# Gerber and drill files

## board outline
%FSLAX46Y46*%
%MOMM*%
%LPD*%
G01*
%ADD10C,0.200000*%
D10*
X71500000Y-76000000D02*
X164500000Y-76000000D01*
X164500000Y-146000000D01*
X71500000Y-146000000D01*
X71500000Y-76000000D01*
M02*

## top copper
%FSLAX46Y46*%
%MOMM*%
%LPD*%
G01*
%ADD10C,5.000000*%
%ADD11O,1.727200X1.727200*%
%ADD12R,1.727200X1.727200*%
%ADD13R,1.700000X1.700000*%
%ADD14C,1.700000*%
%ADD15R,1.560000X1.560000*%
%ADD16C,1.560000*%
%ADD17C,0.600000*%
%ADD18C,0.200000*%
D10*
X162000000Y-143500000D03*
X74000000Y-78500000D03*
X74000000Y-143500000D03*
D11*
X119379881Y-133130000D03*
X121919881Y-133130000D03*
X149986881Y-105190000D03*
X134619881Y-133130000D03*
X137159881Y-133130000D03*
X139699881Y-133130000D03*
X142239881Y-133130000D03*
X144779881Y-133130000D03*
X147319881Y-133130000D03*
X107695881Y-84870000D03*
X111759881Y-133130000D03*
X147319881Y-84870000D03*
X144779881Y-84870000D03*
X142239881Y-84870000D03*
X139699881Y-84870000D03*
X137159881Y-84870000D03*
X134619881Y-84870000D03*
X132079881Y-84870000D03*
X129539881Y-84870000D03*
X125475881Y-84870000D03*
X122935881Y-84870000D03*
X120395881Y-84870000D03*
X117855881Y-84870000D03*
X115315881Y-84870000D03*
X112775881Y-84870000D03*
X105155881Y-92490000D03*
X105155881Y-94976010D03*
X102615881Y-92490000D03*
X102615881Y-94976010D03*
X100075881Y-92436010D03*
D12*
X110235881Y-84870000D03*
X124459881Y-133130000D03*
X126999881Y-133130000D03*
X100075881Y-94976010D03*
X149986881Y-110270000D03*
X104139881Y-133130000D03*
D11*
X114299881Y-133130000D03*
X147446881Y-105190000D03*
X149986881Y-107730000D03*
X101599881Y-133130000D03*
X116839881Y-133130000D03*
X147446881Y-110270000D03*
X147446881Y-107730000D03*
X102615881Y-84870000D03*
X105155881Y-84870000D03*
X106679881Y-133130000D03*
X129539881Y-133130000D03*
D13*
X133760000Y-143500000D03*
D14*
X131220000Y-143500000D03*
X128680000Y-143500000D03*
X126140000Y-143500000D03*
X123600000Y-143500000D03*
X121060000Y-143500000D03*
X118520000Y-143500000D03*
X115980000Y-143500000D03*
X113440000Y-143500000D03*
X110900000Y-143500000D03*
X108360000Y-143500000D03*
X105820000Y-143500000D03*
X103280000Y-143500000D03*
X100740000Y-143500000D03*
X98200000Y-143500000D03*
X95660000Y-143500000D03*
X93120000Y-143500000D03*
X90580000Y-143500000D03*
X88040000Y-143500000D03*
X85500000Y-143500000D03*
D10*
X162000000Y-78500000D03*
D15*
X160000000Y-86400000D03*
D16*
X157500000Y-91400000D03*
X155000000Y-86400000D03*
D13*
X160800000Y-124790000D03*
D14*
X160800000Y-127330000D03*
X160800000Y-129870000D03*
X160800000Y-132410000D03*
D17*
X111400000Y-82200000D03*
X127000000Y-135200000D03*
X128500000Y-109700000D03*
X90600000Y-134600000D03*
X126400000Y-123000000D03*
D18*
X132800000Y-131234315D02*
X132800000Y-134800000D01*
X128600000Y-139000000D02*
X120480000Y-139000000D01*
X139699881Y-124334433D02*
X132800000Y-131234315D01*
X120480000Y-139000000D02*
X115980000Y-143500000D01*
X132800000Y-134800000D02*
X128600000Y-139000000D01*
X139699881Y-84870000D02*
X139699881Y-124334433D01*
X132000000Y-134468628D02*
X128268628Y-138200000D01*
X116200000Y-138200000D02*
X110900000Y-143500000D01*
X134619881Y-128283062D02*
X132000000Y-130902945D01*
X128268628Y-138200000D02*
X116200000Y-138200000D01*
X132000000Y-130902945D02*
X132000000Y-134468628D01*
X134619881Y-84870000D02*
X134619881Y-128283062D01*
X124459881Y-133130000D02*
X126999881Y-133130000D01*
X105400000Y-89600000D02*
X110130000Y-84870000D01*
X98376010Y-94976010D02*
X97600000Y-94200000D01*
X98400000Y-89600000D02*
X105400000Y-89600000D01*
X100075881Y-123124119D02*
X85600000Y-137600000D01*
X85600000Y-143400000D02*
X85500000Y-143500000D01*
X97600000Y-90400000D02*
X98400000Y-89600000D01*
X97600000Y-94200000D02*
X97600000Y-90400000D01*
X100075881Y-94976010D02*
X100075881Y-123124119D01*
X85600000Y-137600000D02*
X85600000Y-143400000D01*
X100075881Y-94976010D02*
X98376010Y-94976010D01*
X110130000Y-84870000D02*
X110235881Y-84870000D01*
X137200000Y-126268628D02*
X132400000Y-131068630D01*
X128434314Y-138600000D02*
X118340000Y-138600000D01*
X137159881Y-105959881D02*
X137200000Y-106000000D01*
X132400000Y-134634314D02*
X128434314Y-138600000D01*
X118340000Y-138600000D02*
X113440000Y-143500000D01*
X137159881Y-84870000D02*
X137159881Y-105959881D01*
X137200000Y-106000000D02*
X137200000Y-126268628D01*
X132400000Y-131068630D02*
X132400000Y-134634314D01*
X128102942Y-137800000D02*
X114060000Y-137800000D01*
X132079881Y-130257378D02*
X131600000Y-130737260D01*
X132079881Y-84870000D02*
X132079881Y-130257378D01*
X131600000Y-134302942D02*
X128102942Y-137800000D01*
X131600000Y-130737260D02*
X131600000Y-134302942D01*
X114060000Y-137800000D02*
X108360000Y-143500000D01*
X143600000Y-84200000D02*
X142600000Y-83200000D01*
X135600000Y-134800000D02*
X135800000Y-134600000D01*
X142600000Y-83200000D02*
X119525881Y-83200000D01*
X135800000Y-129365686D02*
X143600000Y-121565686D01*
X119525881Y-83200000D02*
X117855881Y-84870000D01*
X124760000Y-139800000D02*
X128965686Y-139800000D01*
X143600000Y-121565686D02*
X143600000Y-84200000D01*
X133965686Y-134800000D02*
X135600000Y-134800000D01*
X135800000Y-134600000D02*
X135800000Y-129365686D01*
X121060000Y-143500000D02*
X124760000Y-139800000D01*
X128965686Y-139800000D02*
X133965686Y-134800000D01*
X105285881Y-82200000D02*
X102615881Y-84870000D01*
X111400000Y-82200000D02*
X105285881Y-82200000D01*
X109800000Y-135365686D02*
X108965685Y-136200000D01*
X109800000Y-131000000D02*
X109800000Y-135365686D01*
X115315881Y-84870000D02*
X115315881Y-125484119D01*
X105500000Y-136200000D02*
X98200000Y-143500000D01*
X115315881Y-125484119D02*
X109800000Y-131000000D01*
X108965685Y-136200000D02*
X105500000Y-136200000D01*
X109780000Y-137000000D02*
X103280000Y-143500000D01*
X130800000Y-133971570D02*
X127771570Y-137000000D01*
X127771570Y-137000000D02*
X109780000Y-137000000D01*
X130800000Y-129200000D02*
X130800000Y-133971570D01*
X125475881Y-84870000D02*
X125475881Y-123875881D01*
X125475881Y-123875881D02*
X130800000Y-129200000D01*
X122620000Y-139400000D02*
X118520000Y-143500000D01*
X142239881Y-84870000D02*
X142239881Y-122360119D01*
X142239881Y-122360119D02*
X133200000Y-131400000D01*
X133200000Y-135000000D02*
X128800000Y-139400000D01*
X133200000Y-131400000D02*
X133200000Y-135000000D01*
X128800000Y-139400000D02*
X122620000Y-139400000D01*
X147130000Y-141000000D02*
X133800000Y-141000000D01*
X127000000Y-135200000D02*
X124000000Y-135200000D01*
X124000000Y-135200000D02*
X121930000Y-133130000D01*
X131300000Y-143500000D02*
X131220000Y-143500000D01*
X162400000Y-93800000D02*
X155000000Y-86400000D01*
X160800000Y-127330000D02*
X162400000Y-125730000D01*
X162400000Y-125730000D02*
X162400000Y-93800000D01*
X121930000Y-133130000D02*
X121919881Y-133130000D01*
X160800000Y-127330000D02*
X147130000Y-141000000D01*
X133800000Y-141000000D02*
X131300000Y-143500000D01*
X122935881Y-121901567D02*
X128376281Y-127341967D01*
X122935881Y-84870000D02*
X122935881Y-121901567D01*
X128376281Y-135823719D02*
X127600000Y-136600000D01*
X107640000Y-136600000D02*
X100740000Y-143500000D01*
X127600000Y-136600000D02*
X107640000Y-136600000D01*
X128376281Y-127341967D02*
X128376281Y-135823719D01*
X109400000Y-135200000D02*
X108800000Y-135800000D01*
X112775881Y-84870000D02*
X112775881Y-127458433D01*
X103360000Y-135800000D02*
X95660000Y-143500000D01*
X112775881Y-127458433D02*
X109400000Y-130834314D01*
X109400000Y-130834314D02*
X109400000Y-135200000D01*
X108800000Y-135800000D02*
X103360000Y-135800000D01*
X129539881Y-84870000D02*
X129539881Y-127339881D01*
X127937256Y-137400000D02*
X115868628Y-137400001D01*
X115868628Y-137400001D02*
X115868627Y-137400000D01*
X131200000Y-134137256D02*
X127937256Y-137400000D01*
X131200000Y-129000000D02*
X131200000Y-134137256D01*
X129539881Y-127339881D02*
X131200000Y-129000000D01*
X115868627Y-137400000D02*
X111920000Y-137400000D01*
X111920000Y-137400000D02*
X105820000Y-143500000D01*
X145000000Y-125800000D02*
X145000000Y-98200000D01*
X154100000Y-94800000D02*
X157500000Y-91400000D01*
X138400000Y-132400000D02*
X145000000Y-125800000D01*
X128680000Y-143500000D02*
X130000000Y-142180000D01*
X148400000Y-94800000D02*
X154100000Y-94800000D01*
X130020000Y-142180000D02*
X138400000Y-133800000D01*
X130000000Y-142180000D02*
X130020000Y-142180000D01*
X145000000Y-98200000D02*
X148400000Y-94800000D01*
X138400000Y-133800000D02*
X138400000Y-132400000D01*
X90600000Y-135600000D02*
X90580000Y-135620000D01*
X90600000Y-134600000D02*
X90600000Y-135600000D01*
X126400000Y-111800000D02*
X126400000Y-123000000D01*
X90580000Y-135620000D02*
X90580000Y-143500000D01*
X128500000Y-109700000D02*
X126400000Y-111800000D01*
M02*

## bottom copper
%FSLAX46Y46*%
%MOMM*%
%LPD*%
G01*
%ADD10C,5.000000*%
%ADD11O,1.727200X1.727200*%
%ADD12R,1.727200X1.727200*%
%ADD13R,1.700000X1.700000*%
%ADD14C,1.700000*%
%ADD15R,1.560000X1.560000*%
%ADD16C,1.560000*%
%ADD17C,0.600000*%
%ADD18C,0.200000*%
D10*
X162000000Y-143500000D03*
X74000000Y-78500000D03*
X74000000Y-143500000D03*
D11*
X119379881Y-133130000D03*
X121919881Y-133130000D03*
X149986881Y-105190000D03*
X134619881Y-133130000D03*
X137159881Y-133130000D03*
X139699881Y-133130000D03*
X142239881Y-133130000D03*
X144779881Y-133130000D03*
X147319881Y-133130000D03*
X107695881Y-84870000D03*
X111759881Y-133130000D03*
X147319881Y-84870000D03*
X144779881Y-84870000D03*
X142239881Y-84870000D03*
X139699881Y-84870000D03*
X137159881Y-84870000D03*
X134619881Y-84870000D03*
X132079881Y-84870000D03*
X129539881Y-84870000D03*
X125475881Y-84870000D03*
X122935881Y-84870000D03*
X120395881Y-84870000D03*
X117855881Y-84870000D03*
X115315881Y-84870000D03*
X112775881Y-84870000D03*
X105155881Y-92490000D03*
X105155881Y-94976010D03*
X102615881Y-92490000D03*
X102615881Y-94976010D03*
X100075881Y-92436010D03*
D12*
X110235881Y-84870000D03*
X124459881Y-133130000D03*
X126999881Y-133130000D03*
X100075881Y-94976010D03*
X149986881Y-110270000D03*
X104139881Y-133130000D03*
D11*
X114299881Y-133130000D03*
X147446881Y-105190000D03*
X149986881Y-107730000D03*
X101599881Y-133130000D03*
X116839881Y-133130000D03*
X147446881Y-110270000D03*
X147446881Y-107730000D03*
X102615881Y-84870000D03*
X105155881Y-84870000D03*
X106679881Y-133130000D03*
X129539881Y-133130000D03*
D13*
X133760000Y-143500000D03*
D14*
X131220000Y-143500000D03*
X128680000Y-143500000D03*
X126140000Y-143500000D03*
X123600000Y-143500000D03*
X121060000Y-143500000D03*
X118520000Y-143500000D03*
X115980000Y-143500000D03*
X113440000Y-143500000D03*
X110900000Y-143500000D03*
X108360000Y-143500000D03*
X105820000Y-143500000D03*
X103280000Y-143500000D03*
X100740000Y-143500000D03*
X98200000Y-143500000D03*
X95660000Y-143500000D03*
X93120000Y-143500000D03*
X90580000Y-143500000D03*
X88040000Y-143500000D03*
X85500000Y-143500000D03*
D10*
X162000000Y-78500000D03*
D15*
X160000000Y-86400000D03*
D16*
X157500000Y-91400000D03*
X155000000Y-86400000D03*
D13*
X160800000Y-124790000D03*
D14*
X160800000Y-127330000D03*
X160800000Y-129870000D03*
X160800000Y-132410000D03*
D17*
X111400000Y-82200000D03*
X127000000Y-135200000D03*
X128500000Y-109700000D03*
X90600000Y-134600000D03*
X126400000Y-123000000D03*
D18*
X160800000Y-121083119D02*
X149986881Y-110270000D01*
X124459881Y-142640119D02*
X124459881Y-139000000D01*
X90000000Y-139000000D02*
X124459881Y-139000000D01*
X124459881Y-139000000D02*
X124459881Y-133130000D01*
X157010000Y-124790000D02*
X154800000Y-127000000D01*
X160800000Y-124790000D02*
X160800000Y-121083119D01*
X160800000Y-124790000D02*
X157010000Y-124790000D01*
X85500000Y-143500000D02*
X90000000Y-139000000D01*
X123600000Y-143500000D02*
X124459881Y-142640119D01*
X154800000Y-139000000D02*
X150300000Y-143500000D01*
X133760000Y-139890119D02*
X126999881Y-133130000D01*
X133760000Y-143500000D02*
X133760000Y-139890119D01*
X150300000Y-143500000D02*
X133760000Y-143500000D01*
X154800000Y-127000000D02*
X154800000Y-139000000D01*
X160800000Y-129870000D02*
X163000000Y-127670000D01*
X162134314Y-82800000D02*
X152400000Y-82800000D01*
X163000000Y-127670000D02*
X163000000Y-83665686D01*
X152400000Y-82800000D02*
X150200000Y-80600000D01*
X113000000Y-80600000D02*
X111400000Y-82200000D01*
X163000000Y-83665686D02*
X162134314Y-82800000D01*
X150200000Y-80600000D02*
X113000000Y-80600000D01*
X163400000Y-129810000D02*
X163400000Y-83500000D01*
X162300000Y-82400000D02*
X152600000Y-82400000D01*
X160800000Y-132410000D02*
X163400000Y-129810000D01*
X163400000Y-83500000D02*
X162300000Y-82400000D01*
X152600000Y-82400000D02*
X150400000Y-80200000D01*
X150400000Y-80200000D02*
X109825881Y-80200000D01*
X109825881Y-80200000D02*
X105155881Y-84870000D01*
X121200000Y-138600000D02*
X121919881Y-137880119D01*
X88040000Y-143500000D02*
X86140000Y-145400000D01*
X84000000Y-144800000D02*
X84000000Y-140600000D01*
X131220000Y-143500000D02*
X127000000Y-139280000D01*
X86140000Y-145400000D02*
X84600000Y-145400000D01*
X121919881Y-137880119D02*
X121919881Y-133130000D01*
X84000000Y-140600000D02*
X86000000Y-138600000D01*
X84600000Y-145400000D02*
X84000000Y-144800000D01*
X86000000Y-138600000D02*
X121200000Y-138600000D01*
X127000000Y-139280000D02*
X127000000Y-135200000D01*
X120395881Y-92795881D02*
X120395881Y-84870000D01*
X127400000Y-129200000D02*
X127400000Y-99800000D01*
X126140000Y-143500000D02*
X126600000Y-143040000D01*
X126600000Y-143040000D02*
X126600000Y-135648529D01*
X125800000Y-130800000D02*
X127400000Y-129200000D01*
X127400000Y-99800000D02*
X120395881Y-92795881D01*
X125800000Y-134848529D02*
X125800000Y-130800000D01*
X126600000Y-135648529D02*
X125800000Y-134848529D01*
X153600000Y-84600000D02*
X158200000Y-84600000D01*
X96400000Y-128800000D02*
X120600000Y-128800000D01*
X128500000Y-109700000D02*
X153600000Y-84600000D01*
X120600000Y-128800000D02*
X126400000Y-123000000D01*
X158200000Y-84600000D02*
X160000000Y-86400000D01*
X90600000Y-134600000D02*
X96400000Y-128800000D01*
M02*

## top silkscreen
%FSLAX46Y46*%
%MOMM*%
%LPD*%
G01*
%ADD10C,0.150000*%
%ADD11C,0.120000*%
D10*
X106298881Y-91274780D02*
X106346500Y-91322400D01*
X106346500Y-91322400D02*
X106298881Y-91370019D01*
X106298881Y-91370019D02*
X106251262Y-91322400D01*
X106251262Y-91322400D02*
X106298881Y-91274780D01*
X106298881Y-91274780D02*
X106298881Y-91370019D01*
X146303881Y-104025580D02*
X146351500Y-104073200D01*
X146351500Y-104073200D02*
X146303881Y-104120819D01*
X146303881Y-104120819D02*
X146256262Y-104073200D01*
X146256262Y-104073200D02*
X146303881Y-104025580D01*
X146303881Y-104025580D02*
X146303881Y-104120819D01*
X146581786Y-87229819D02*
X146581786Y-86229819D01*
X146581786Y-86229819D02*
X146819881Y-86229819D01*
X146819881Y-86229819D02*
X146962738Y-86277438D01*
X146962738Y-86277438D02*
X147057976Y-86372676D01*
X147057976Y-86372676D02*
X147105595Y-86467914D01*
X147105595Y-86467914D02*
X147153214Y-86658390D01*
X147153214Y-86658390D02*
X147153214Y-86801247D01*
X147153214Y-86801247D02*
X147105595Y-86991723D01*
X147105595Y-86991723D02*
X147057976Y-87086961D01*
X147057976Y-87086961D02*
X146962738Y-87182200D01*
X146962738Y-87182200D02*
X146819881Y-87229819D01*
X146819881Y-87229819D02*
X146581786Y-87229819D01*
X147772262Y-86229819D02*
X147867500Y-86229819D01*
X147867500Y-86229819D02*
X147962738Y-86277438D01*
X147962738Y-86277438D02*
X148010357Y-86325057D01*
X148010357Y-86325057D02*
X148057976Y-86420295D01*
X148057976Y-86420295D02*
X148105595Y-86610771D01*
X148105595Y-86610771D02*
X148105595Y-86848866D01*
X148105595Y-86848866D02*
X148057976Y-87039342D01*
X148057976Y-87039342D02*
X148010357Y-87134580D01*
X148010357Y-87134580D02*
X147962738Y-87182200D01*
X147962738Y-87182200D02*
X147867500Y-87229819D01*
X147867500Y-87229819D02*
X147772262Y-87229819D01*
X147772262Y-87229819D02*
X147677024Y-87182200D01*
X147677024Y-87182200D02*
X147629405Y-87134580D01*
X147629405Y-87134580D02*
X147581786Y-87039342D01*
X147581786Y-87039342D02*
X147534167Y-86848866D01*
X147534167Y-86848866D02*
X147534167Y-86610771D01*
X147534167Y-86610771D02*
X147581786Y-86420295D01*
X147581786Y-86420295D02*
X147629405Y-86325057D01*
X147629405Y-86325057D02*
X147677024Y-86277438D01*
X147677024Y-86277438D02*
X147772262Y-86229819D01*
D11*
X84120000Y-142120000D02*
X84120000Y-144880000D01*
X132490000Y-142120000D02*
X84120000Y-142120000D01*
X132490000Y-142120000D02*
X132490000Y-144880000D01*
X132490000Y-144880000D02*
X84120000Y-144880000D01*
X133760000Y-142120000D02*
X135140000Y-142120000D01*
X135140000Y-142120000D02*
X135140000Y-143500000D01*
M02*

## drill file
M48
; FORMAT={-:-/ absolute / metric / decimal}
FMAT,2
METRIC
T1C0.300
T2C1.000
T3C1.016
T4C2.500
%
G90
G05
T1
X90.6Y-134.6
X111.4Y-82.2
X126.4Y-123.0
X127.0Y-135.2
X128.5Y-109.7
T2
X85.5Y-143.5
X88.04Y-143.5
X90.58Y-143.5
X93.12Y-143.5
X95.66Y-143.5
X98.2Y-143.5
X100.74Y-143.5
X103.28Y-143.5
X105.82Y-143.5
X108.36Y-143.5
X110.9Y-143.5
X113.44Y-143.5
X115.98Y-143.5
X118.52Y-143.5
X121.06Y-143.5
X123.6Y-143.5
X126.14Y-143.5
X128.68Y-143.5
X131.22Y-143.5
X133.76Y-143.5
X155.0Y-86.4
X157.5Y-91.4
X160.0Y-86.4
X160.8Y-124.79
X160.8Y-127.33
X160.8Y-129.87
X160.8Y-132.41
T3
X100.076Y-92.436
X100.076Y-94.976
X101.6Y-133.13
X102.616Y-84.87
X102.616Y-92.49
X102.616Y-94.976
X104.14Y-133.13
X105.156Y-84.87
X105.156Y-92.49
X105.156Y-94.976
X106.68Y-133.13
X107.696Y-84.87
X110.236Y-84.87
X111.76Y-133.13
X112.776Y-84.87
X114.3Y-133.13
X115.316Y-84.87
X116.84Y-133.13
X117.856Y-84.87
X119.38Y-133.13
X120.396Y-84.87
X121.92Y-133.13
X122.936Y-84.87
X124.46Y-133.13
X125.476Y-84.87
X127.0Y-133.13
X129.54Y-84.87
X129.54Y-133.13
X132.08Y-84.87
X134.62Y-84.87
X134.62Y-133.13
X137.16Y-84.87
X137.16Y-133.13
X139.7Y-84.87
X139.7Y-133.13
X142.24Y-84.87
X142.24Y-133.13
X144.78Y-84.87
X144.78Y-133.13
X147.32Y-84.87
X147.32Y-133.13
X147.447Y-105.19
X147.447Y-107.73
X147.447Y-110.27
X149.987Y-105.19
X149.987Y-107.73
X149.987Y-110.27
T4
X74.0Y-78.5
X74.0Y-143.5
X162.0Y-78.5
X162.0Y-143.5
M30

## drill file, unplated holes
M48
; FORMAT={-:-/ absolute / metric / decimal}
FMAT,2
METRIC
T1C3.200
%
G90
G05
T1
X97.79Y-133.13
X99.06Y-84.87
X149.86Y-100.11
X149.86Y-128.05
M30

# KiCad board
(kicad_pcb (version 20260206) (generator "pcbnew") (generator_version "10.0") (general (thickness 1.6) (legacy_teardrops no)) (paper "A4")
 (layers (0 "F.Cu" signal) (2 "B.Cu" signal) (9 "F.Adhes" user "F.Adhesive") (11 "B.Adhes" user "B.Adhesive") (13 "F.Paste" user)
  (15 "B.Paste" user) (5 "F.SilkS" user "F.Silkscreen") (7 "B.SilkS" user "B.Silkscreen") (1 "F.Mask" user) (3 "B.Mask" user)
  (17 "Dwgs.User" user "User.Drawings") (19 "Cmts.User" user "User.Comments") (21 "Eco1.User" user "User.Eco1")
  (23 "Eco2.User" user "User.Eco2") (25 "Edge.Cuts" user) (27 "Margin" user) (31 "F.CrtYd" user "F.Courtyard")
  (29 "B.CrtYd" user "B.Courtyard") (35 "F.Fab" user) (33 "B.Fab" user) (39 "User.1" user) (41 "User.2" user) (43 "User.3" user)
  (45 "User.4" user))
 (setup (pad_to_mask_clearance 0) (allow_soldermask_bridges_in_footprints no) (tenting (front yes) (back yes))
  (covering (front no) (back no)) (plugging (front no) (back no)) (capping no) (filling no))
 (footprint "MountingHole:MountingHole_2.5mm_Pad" (layer "F.Cu") (at 162 143.5)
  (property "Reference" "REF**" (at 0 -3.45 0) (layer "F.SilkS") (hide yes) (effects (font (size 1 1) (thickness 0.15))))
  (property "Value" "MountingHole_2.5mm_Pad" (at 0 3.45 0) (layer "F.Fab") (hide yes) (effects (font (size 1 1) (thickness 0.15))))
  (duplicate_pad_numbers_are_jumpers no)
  (pad "1" thru_hole circle (at 0 0) (size 5 5) (drill 2.5) (layers "*.Cu" "*.Mask") (remove_unused_layers no) (zone_connect 2)))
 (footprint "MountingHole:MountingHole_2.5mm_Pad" (layer "F.Cu") (at 74 78.5)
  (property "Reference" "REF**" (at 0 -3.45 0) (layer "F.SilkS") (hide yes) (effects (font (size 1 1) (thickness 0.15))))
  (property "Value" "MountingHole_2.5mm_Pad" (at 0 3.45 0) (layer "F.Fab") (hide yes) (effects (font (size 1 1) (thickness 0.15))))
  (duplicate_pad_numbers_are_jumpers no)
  (pad "1" thru_hole circle (at 0 0) (size 5 5) (drill 2.5) (layers "*.Cu" "*.Mask") (remove_unused_layers no) (zone_connect 2)))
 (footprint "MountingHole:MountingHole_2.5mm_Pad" (layer "F.Cu") (at 74 143.5)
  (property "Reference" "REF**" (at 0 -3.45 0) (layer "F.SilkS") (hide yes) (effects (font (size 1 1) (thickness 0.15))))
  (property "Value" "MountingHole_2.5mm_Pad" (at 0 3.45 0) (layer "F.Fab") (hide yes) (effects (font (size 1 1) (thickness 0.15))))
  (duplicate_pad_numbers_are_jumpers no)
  (pad "1" thru_hole circle (at 0 0) (size 5 5) (drill 2.5) (layers "*.Cu" "*.Mask") (remove_unused_layers no) (zone_connect 2)))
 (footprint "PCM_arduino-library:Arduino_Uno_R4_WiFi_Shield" (layer "F.Cu") (at 83.819881 135.67)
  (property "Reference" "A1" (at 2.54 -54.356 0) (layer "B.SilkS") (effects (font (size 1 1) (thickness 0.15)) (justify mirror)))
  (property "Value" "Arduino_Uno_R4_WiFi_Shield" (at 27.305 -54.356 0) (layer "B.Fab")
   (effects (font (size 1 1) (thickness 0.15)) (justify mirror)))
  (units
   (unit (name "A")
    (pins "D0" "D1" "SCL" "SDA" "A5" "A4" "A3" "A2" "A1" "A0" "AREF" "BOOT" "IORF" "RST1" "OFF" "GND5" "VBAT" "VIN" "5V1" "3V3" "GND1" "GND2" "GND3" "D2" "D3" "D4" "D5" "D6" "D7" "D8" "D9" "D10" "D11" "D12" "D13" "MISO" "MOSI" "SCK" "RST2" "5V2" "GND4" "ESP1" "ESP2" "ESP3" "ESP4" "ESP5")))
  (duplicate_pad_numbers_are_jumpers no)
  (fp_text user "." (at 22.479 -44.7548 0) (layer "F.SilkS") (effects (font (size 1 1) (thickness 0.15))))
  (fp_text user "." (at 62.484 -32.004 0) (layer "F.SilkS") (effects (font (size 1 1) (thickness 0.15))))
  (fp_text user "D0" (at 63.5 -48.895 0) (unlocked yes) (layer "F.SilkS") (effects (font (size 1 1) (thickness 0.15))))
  (pad "" np_thru_hole circle (at 13.97 -2.54) (size 3.2 3.2) (drill 3.2) (layers "*.Cu" "*.Mask"))
  (pad "" np_thru_hole circle (at 15.24 -50.8) (size 3.2 3.2) (drill 3.2) (layers "*.Cu" "*.Mask"))
  (pad "" np_thru_hole circle (at 66.04 -35.56) (size 3.2 3.2) (drill 3.2) (layers "*.Cu" "*.Mask"))
  (pad "" np_thru_hole circle (at 66.04 -7.62) (size 3.2 3.2) (drill 3.2) (layers "*.Cu" "*.Mask"))
  (pad "3V3" thru_hole oval (at 35.56 -2.54) (size 1.7272 1.7272) (drill 1.016) (layers "*.Cu" "*.Mask") (remove_unused_layers no)
   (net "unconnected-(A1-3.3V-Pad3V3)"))
  (pad "5V1" thru_hole oval (at 38.1 -2.54) (size 1.7272 1.7272) (drill 1.016) (layers "*.Cu" "*.Mask") (remove_unused_layers no)
   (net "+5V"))
  (pad "5V2" thru_hole oval (at 66.167 -30.48) (size 1.7272 1.7272) (drill 1.016) (layers "*.Cu" "*.Mask") (remove_unused_layers no)
   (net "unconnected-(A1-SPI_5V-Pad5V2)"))
  (pad "A0" thru_hole oval (at 50.8 -2.54) (size 1.7272 1.7272) (drill 1.016) (layers "*.Cu" "*.Mask") (remove_unused_layers no)
   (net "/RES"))
  (pad "A1" thru_hole oval (at 53.34 -2.54) (size 1.7272 1.7272) (drill 1.016) (layers "*.Cu" "*.Mask") (remove_unused_layers no)
   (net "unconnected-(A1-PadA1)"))
  (pad "A2" thru_hole oval (at 55.88 -2.54) (size 1.7272 1.7272) (drill 1.016) (layers "*.Cu" "*.Mask") (remove_unused_layers no)
   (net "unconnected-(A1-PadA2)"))
  (pad "A3" thru_hole oval (at 58.42 -2.54) (size 1.7272 1.7272) (drill 1.016) (layers "*.Cu" "*.Mask") (remove_unused_layers no)
   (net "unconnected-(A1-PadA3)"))
  (pad "A4" thru_hole oval (at 60.96 -2.54) (size 1.7272 1.7272) (drill 1.016) (layers "*.Cu" "*.Mask") (remove_unused_layers no)
   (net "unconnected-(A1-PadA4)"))
  (pad "A5" thru_hole oval (at 63.5 -2.54) (size 1.7272 1.7272) (drill 1.016) (layers "*.Cu" "*.Mask") (remove_unused_layers no)
   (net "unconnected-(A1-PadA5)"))
  (pad "AREF" thru_hole oval (at 23.876 -50.8) (size 1.7272 1.7272) (drill 1.016) (layers "*.Cu" "*.Mask") (remove_unused_layers no)
   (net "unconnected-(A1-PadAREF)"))
  (pad "BOOT" thru_hole oval (at 27.94 -2.54) (size 1.7272 1.7272) (drill 1.016) (layers "*.Cu" "*.Mask") (remove_unused_layers no)
   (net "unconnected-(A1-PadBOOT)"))
  (pad "D0" thru_hole oval (at 63.5 -50.8) (size 1.7272 1.7272) (drill 1.016) (layers "*.Cu" "*.Mask") (remove_unused_layers no)
   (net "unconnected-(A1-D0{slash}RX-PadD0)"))
  (pad "D1" thru_hole oval (at 60.96 -50.8) (size 1.7272 1.7272) (drill 1.016) (layers "*.Cu" "*.Mask") (remove_unused_layers no)
   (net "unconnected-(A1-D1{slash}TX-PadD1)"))
  (pad "D2" thru_hole oval (at 58.42 -50.8) (size 1.7272 1.7272) (drill 1.016) (layers "*.Cu" "*.Mask") (remove_unused_layers no)
   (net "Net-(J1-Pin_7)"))
  (pad "D3" thru_hole oval (at 55.88 -50.8) (size 1.7272 1.7272) (drill 1.016) (layers "*.Cu" "*.Mask") (remove_unused_layers no)
   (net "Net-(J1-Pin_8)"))
  (pad "D4" thru_hole oval (at 53.34 -50.8) (size 1.7272 1.7272) (drill 1.016) (layers "*.Cu" "*.Mask") (remove_unused_layers no)
   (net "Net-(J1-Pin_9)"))
  (pad "D5" thru_hole oval (at 50.8 -50.8) (size 1.7272 1.7272) (drill 1.016) (layers "*.Cu" "*.Mask") (remove_unused_layers no)
   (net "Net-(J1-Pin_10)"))
  (pad "D6" thru_hole oval (at 48.26 -50.8) (size 1.7272 1.7272) (drill 1.016) (layers "*.Cu" "*.Mask") (remove_unused_layers no)
   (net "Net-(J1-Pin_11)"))
  (pad "D7" thru_hole oval (at 45.72 -50.8) (size 1.7272 1.7272) (drill 1.016) (layers "*.Cu" "*.Mask") (remove_unused_layers no)
   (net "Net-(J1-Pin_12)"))
  (pad "D8" thru_hole oval (at 41.656 -50.8) (size 1.7272 1.7272) (drill 1.016) (layers "*.Cu" "*.Mask") (remove_unused_layers no)
   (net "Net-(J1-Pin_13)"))
  (pad "D9" thru_hole oval (at 39.116 -50.8) (size 1.7272 1.7272) (drill 1.016) (layers "*.Cu" "*.Mask") (remove_unused_layers no)
   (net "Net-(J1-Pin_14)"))
  (pad "D10" thru_hole oval (at 36.576 -50.8) (size 1.7272 1.7272) (drill 1.016) (layers "*.Cu" "*.Mask") (remove_unused_layers no)
   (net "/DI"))
  (pad "D11" thru_hole oval (at 34.036 -50.8) (size 1.7272 1.7272) (drill 1.016) (layers "*.Cu" "*.Mask") (remove_unused_layers no)
   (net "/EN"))
  (pad "D12" thru_hole oval (at 31.496 -50.8) (size 1.7272 1.7272) (drill 1.016) (layers "*.Cu" "*.Mask") (remove_unused_layers no)
   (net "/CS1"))
  (pad "D13" thru_hole oval (at 28.956 -50.8) (size 1.7272 1.7272) (drill 1.016) (layers "*.Cu" "*.Mask") (remove_unused_layers no)
   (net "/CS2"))
  (pad "ESP1" thru_hole oval (at 21.336 -43.18) (size 1.7272 1.7272) (drill 1.016) (layers "*.Cu" "*.Mask") (remove_unused_layers no)
   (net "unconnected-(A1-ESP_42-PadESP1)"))
  (pad "ESP2" thru_hole oval (at 21.336 -40.69399) (size 1.7272 1.7272) (drill 1.016) (layers "*.Cu" "*.Mask") (remove_unused_layers no)
   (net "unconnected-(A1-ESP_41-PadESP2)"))
  (pad "ESP3" thru_hole oval (at 18.796 -43.18) (size 1.7272 1.7272) (drill 1.016) (layers "*.Cu" "*.Mask") (remove_unused_layers no)
   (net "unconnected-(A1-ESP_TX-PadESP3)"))
  (pad "ESP4" thru_hole oval (at 18.796 -40.69399) (size 1.7272 1.7272) (drill 1.016) (layers "*.Cu" "*.Mask") (remove_unused_layers no)
   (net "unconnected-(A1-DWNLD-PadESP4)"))
  (pad "ESP5" thru_hole oval (at 16.256 -43.23399) (size 1.7272 1.7272) (drill 1.016) (layers "*.Cu" "*.Mask") (remove_unused_layers no)
   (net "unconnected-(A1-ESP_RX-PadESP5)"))
  (pad "GND1" thru_hole rect (at 26.416 -50.8) (size 1.7272 1.7272) (drill 1.016) (layers "*.Cu" "*.Mask") (remove_unused_layers no)
   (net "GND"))
  (pad "GND2" thru_hole rect (at 40.64 -2.54) (size 1.7272 1.7272) (drill 1.016) (layers "*.Cu" "*.Mask") (remove_unused_layers no)
   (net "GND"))
  (pad "GND3" thru_hole rect (at 43.18 -2.54) (size 1.7272 1.7272) (drill 1.016) (layers "*.Cu" "*.Mask") (remove_unused_layers no)
   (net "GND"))
  (pad "GND4" thru_hole rect (at 16.256 -40.69399) (size 1.7272 1.7272) (drill 1.016) (layers "*.Cu" "*.Mask") (remove_unused_layers no)
   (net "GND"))
  (pad "GND4" thru_hole rect (at 66.167 -25.4) (size 1.7272 1.7272) (drill 1.016) (layers "*.Cu" "*.Mask") (remove_unused_layers no)
   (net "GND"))
  (pad "GND5" thru_hole rect (at 20.32 -2.54) (size 1.7272 1.7272) (drill 1.016) (layers "*.Cu" "*.Mask") (remove_unused_layers no)
   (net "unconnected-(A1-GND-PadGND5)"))
  (pad "IORF" thru_hole oval (at 30.48 -2.54) (size 1.7272 1.7272) (drill 1.016) (layers "*.Cu" "*.Mask") (remove_unused_layers no)
   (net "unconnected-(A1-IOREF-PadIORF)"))
  (pad "MISO" thru_hole oval (at 63.627 -30.48) (size 1.7272 1.7272) (drill 1.016) (layers "*.Cu" "*.Mask") (remove_unused_layers no)
   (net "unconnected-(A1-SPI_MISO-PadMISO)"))
  (pad "MOSI" thru_hole oval (at 66.167 -27.94) (size 1.7272 1.7272) (drill 1.016) (layers "*.Cu" "*.Mask") (remove_unused_layers no)
   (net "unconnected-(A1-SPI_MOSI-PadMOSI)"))
  (pad "OFF" thru_hole oval (at 17.78 -2.54) (size 1.7272 1.7272) (drill 1.016) (layers "*.Cu" "*.Mask") (remove_unused_layers no)
   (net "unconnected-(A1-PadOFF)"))
  (pad "RST1" thru_hole oval (at 33.02 -2.54) (size 1.7272 1.7272) (drill 1.016) (layers "*.Cu" "*.Mask") (remove_unused_layers no)
   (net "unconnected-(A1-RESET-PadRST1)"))
  (pad "RST2" thru_hole oval (at 63.627 -25.4) (size 1.7272 1.7272) (drill 1.016) (layers "*.Cu" "*.Mask") (remove_unused_layers no)
   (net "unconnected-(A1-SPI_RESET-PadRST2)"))
  (pad "SCK" thru_hole oval (at 63.627 -27.94) (size 1.7272 1.7272) (drill 1.016) (layers "*.Cu" "*.Mask") (remove_unused_layers no)
   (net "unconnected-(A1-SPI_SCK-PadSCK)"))
  (pad "SCL" thru_hole oval (at 18.796 -50.8) (size 1.7272 1.7272) (drill 1.016) (layers "*.Cu" "*.Mask") (remove_unused_layers no)
   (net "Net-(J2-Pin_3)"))
  (pad "SDA" thru_hole oval (at 21.336 -50.8) (size 1.7272 1.7272) (drill 1.016) (layers "*.Cu" "*.Mask") (remove_unused_layers no)
   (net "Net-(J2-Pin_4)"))
  (pad "VBAT" thru_hole oval (at 22.86 -2.54) (size 1.7272 1.7272) (drill 1.016) (layers "*.Cu" "*.Mask") (remove_unused_layers no)
   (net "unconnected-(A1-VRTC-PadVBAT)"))
  (pad "VIN" thru_hole oval (at 45.72 -2.54) (size 1.7272 1.7272) (drill 1.016) (layers "*.Cu" "*.Mask") (remove_unused_layers no)
   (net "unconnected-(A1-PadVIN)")))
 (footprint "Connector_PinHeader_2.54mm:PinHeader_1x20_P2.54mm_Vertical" (layer "F.Cu") (at 133.76 143.5 -90)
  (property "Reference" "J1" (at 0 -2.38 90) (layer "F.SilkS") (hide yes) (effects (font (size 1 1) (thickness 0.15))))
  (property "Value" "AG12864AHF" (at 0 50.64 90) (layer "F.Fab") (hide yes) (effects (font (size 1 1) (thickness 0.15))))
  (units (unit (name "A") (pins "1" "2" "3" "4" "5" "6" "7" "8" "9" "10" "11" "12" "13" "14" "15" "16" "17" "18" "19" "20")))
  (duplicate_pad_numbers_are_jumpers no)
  (fp_line (start -1.38 49.64) (end 1.38 49.64) (stroke (width 0.12) (type solid)) (layer "F.SilkS"))
  (fp_line (start -1.38 1.27) (end -1.38 49.64) (stroke (width 0.12) (type solid)) (layer "F.SilkS"))
  (fp_line (start -1.38 1.27) (end 1.38 1.27) (stroke (width 0.12) (type solid)) (layer "F.SilkS"))
  (fp_line (start 1.38 1.27) (end 1.38 49.64) (stroke (width 0.12) (type solid)) (layer "F.SilkS"))
  (fp_line (start -1.38 0) (end -1.38 -1.38) (stroke (width 0.12) (type solid)) (layer "F.SilkS"))
  (fp_line (start -1.38 -1.38) (end 0 -1.38) (stroke (width 0.12) (type solid)) (layer "F.SilkS"))
  (pad "1" thru_hole rect (at 0 0 270) (size 1.7 1.7) (drill 1) (layers "*.Cu" "*.Mask") (remove_unused_layers no) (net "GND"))
  (pad "2" thru_hole circle (at 0 2.54 270) (size 1.7 1.7) (drill 1) (layers "*.Cu" "*.Mask") (remove_unused_layers no) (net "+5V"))
  (pad "3" thru_hole circle (at 0 5.08 270) (size 1.7 1.7) (drill 1) (layers "*.Cu" "*.Mask") (remove_unused_layers no) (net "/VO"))
  (pad "4" thru_hole circle (at 0 7.62 270) (size 1.7 1.7) (drill 1) (layers "*.Cu" "*.Mask") (remove_unused_layers no) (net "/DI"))
  (pad "5" thru_hole circle (at 0 10.16 270) (size 1.7 1.7) (drill 1) (layers "*.Cu" "*.Mask") (remove_unused_layers no) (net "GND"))
  (pad "6" thru_hole circle (at 0 12.7 270) (size 1.7 1.7) (drill 1) (layers "*.Cu" "*.Mask") (remove_unused_layers no) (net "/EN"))
  (pad "7" thru_hole circle (at 0 15.24 270) (size 1.7 1.7) (drill 1) (layers "*.Cu" "*.Mask") (remove_unused_layers no)
   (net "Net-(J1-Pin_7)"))
  (pad "8" thru_hole circle (at 0 17.78 270) (size 1.7 1.7) (drill 1) (layers "*.Cu" "*.Mask") (remove_unused_layers no)
   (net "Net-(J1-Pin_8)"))
  (pad "9" thru_hole circle (at 0 20.32 270) (size 1.7 1.7) (drill 1) (layers "*.Cu" "*.Mask") (remove_unused_layers no)
   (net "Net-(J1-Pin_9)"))
  (pad "10" thru_hole circle (at 0 22.86 270) (size 1.7 1.7) (drill 1) (layers "*.Cu" "*.Mask") (remove_unused_layers no)
   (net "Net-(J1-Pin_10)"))
  (pad "11" thru_hole circle (at 0 25.4 270) (size 1.7 1.7) (drill 1) (layers "*.Cu" "*.Mask") (remove_unused_layers no)
   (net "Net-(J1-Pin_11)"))
  (pad "12" thru_hole circle (at 0 27.94 270) (size 1.7 1.7) (drill 1) (layers "*.Cu" "*.Mask") (remove_unused_layers no)
   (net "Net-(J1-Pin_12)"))
  (pad "13" thru_hole circle (at 0 30.48 270) (size 1.7 1.7) (drill 1) (layers "*.Cu" "*.Mask") (remove_unused_layers no)
   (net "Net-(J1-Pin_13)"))
  (pad "14" thru_hole circle (at 0 33.02 270) (size 1.7 1.7) (drill 1) (layers "*.Cu" "*.Mask") (remove_unused_layers no)
   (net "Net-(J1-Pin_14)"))
  (pad "15" thru_hole circle (at 0 35.56 270) (size 1.7 1.7) (drill 1) (layers "*.Cu" "*.Mask") (remove_unused_layers no) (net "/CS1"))
  (pad "16" thru_hole circle (at 0 38.1 270) (size 1.7 1.7) (drill 1) (layers "*.Cu" "*.Mask") (remove_unused_layers no) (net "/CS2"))
  (pad "17" thru_hole circle (at 0 40.64 270) (size 1.7 1.7) (drill 1) (layers "*.Cu" "*.Mask") (remove_unused_layers no) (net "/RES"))
  (pad "18" thru_hole circle (at 0 43.18 270) (size 1.7 1.7) (drill 1) (layers "*.Cu" "*.Mask") (remove_unused_layers no) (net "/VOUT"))
  (pad "19" thru_hole circle (at 0 45.72 270) (size 1.7 1.7) (drill 1) (layers "*.Cu" "*.Mask") (remove_unused_layers no) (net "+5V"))
  (pad "20" thru_hole circle (at 0 48.26 270) (size 1.7 1.7) (drill 1) (layers "*.Cu" "*.Mask") (remove_unused_layers no) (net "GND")))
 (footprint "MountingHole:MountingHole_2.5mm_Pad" (layer "F.Cu") (at 162 78.5)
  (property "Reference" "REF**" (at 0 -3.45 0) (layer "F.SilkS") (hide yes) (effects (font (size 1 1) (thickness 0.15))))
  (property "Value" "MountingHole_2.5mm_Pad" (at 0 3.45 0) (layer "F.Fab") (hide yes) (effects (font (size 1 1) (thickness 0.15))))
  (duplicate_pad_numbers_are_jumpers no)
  (pad "1" thru_hole circle (at 0 0) (size 5 5) (drill 2.5) (layers "*.Cu" "*.Mask") (remove_unused_layers no) (zone_connect 2)))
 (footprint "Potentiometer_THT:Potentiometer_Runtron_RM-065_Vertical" (layer "B.Cu") (at 160 86.4 180)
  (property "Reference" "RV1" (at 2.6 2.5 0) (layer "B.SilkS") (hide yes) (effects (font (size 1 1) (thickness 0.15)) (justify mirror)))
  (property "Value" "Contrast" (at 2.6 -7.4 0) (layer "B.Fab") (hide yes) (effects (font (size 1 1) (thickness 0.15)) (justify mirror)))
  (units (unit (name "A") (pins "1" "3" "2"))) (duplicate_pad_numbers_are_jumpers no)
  (pad "1" thru_hole rect (at 0 0 180) (size 1.56 1.56) (drill 1) (layers "*.Cu" "*.Mask") (remove_unused_layers no) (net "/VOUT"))
  (pad "2" thru_hole circle (at 2.5 -5 180) (size 1.56 1.56) (drill 1) (layers "*.Cu" "*.Mask") (remove_unused_layers no) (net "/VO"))
  (pad "3" thru_hole circle (at 5 0 180) (size 1.56 1.56) (drill 1) (layers "*.Cu" "*.Mask") (remove_unused_layers no) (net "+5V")))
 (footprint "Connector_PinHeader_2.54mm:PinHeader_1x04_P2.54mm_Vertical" (layer "B.Cu") (at 160.8 124.79 180)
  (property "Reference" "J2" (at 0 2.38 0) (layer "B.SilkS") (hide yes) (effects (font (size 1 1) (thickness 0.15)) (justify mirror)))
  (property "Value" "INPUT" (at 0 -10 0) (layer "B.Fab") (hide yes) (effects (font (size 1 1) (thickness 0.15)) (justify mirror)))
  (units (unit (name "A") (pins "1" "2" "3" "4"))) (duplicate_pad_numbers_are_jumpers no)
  (pad "1" thru_hole rect (at 0 0 180) (size 1.7 1.7) (drill 1) (layers "*.Cu" "*.Mask") (remove_unused_layers no) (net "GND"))
  (pad "2" thru_hole circle (at 0 -2.54 180) (size 1.7 1.7) (drill 1) (layers "*.Cu" "*.Mask") (remove_unused_layers no) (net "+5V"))
  (pad "3" thru_hole circle (at 0 -5.08 180) (size 1.7 1.7) (drill 1) (layers "*.Cu" "*.Mask") (remove_unused_layers no)
   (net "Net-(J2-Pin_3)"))
  (pad "4" thru_hole circle (at 0 -7.62 180) (size 1.7 1.7) (drill 1) (layers "*.Cu" "*.Mask") (remove_unused_layers no)
   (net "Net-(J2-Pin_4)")))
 (gr_rect (start 71.5 76) (end 164.5 146) (stroke (width 0.2) (type solid)) (fill no) (layer "Edge.Cuts"))
 (segment (start 147.13 141) (end 133.8 141) (width 0.2) (layer "F.Cu") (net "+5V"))
 (segment (start 127 135.2) (end 124 135.2) (width 0.2) (layer "F.Cu") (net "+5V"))
 (segment (start 124 135.2) (end 121.93 133.13) (width 0.2) (layer "F.Cu") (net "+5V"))
 (segment (start 131.3 143.5) (end 131.22 143.5) (width 0.2) (layer "F.Cu") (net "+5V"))
 (segment (start 162.4 93.8) (end 155 86.4) (width 0.2) (layer "F.Cu") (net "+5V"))
 (segment (start 160.8 127.33) (end 162.4 125.73) (width 0.2) (layer "F.Cu") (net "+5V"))
 (segment (start 162.4 125.73) (end 162.4 93.8) (width 0.2) (layer "F.Cu") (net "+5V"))
 (segment (start 121.93 133.13) (end 121.919881 133.13) (width 0.2) (layer "F.Cu") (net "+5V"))
 (segment (start 160.8 127.33) (end 147.13 141) (width 0.2) (layer "F.Cu") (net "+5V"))
 (segment (start 133.8 141) (end 131.3 143.5) (width 0.2) (layer "F.Cu") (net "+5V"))
 (via (at 127 135.2) (size 0.6) (drill 0.3) (layers "F.Cu" "B.Cu") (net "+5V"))
 (segment (start 121.2 138.6) (end 121.919881 137.880119) (width 0.2) (layer "B.Cu") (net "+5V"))
 (segment (start 88.04 143.5) (end 86.14 145.4) (width 0.2) (layer "B.Cu") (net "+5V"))
 (segment (start 84 144.8) (end 84 140.6) (width 0.2) (layer "B.Cu") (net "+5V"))
 (segment (start 131.22 143.5) (end 127 139.28) (width 0.2) (layer "B.Cu") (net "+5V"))
 (segment (start 86.14 145.4) (end 84.6 145.4) (width 0.2) (layer "B.Cu") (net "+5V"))
 (segment (start 121.919881 137.880119) (end 121.919881 133.13) (width 0.2) (layer "B.Cu") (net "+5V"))
 (segment (start 84 140.6) (end 86 138.6) (width 0.2) (layer "B.Cu") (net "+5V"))
 (segment (start 84.6 145.4) (end 84 144.8) (width 0.2) (layer "B.Cu") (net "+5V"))
 (segment (start 86 138.6) (end 121.2 138.6) (width 0.2) (layer "B.Cu") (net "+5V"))
 (segment (start 127 139.28) (end 127 135.2) (width 0.2) (layer "B.Cu") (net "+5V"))
 (segment (start 122.62 139.4) (end 118.52 143.5) (width 0.2) (layer "F.Cu") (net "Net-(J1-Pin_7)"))
 (segment (start 142.239881 84.87) (end 142.239881 122.360119) (width 0.2) (layer "F.Cu") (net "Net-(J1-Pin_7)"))
 (segment (start 142.239881 122.360119) (end 133.2 131.4) (width 0.2) (layer "F.Cu") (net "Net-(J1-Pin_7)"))
 (segment (start 133.2 135) (end 128.8 139.4) (width 0.2) (layer "F.Cu") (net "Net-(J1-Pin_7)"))
 (segment (start 133.2 131.4) (end 133.2 135) (width 0.2) (layer "F.Cu") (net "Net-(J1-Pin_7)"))
 (segment (start 128.8 139.4) (end 122.62 139.4) (width 0.2) (layer "F.Cu") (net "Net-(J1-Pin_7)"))
 (segment (start 132.8 131.234315) (end 132.8 134.8) (width 0.2) (layer "F.Cu") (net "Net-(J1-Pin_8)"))
 (segment (start 128.6 139) (end 120.48 139) (width 0.2) (layer "F.Cu") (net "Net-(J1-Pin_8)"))
 (segment (start 139.699881 124.334433) (end 132.8 131.234315) (width 0.2) (layer "F.Cu") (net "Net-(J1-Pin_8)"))
 (segment (start 120.48 139) (end 115.98 143.5) (width 0.2) (layer "F.Cu") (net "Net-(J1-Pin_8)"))
 (segment (start 132.8 134.8) (end 128.6 139) (width 0.2) (layer "F.Cu") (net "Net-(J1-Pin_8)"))
 (segment (start 139.699881 84.87) (end 139.699881 124.334433) (width 0.2) (layer "F.Cu") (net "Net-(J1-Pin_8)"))
 (segment (start 137.2 126.268628) (end 132.4 131.06863) (width 0.2) (layer "F.Cu") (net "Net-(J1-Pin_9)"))
 (segment (start 128.434314 138.6) (end 118.34 138.6) (width 0.2) (layer "F.Cu") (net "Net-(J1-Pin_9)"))
 (segment (start 137.159881 105.959881) (end 137.2 106) (width 0.2) (layer "F.Cu") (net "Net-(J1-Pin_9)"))
 (segment (start 132.4 134.634314) (end 128.434314 138.6) (width 0.2) (layer "F.Cu") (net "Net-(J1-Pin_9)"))
 (segment (start 118.34 138.6) (end 113.44 143.5) (width 0.2) (layer "F.Cu") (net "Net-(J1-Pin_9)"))
 (segment (start 137.159881 84.87) (end 137.159881 105.959881) (width 0.2) (layer "F.Cu") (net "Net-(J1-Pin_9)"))
 (segment (start 137.2 106) (end 137.2 126.268628) (width 0.2) (layer "F.Cu") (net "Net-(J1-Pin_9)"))
 (segment (start 132.4 131.06863) (end 132.4 134.634314) (width 0.2) (layer "F.Cu") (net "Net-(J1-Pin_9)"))
 (segment (start 132 134.468628) (end 128.268628 138.2) (width 0.2) (layer "F.Cu") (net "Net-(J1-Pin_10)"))
 (segment (start 116.2 138.2) (end 110.9 143.5) (width 0.2) (layer "F.Cu") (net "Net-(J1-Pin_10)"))
 (segment (start 134.619881 128.283062) (end 132 130.902945) (width 0.2) (layer "F.Cu") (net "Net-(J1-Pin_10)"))
 (segment (start 128.268628 138.2) (end 116.2 138.2) (width 0.2) (layer "F.Cu") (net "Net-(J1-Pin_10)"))
 (segment (start 132 130.902945) (end 132 134.468628) (width 0.2) (layer "F.Cu") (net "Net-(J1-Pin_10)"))
 (segment (start 134.619881 84.87) (end 134.619881 128.283062) (width 0.2) (layer "F.Cu") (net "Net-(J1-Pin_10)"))
 (segment (start 128.102942 137.8) (end 114.06 137.8) (width 0.2) (layer "F.Cu") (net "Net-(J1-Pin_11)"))
 (segment (start 132.079881 130.257378) (end 131.6 130.73726) (width 0.2) (layer "F.Cu") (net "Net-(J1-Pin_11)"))
 (segment (start 132.079881 84.87) (end 132.079881 130.257378) (width 0.2) (layer "F.Cu") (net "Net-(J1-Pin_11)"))
 (segment (start 131.6 134.302942) (end 128.102942 137.8) (width 0.2) (layer "F.Cu") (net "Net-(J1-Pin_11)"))
 (segment (start 131.6 130.73726) (end 131.6 134.302942) (width 0.2) (layer "F.Cu") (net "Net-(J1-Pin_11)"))
 (segment (start 114.06 137.8) (end 108.36 143.5) (width 0.2) (layer "F.Cu") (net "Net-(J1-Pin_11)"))
 (segment (start 129.539881 84.87) (end 129.539881 127.339881) (width 0.2) (layer "F.Cu") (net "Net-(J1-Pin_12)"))
 (segment (start 127.937256 137.4) (end 115.868628 137.400001) (width 0.2) (layer "F.Cu") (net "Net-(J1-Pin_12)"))
 (segment (start 115.868628 137.400001) (end 115.868627 137.4) (width 0.2) (layer "F.Cu") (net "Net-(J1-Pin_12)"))
 (segment (start 131.2 134.137256) (end 127.937256 137.4) (width 0.2) (layer "F.Cu") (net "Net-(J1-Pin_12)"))
 (segment (start 131.2 129) (end 131.2 134.137256) (width 0.2) (layer "F.Cu") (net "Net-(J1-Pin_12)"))
 (segment (start 129.539881 127.339881) (end 131.2 129) (width 0.2) (layer "F.Cu") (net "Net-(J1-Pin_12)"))
 (segment (start 115.868627 137.4) (end 111.92 137.4) (width 0.2) (layer "F.Cu") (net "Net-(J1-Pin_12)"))
 (segment (start 111.92 137.4) (end 105.82 143.5) (width 0.2) (layer "F.Cu") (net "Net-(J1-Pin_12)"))
 (segment (start 109.78 137) (end 103.28 143.5) (width 0.2) (layer "F.Cu") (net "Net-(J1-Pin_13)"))
 (segment (start 130.8 133.97157) (end 127.77157 137) (width 0.2) (layer "F.Cu") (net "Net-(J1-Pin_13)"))
 (segment (start 127.77157 137) (end 109.78 137) (width 0.2) (layer "F.Cu") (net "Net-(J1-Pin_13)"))
 (segment (start 130.8 129.2) (end 130.8 133.97157) (width 0.2) (layer "F.Cu") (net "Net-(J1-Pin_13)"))
 (segment (start 125.475881 84.87) (end 125.475881 123.875881) (width 0.2) (layer "F.Cu") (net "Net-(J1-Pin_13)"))
 (segment (start 125.475881 123.875881) (end 130.8 129.2) (width 0.2) (layer "F.Cu") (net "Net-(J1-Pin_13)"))
 (segment (start 122.935881 121.901567) (end 128.376281 127.341967) (width 0.2) (layer "F.Cu") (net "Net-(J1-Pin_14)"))
 (segment (start 122.935881 84.87) (end 122.935881 121.901567) (width 0.2) (layer "F.Cu") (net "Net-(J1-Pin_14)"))
 (segment (start 128.376281 135.823719) (end 127.6 136.6) (width 0.2) (layer "F.Cu") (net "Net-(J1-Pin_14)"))
 (segment (start 107.64 136.6) (end 100.74 143.5) (width 0.2) (layer "F.Cu") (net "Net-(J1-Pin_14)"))
 (segment (start 127.6 136.6) (end 107.64 136.6) (width 0.2) (layer "F.Cu") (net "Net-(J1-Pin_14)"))
 (segment (start 128.376281 127.341967) (end 128.376281 135.823719) (width 0.2) (layer "F.Cu") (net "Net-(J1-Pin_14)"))
 (segment (start 120.395881 92.795881) (end 120.395881 84.87) (width 0.2) (layer "B.Cu") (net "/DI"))
 (segment (start 127.4 129.2) (end 127.4 99.8) (width 0.2) (layer "B.Cu") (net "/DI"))
 (segment (start 126.14 143.5) (end 126.6 143.04) (width 0.2) (layer "B.Cu") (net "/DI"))
 (segment (start 126.6 143.04) (end 126.6 135.648529) (width 0.2) (layer "B.Cu") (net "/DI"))
 (segment (start 125.8 130.8) (end 127.4 129.2) (width 0.2) (layer "B.Cu") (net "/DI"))
 (segment (start 127.4 99.8) (end 120.395881 92.795881) (width 0.2) (layer "B.Cu") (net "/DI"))
 (segment (start 125.8 134.848529) (end 125.8 130.8) (width 0.2) (layer "B.Cu") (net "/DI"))
 (segment (start 126.6 135.648529) (end 125.8 134.848529) (width 0.2) (layer "B.Cu") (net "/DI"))
 (segment (start 143.6 84.2) (end 142.6 83.2) (width 0.2) (layer "F.Cu") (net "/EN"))
 (segment (start 135.6 134.8) (end 135.8 134.6) (width 0.2) (layer "F.Cu") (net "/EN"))
 (segment (start 142.6 83.2) (end 119.525881 83.2) (width 0.2) (layer "F.Cu") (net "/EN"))
 (segment (start 135.8 129.365686) (end 143.6 121.565686) (width 0.2) (layer "F.Cu") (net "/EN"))
 (segment (start 119.525881 83.2) (end 117.855881 84.87) (width 0.2) (layer "F.Cu") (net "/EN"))
 (segment (start 124.76 139.8) (end 128.965686 139.8) (width 0.2) (layer "F.Cu") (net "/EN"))
 (segment (start 143.6 121.565686) (end 143.6 84.2) (width 0.2) (layer "F.Cu") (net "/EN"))
 (segment (start 133.965686 134.8) (end 135.6 134.8) (width 0.2) (layer "F.Cu") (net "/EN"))
 (segment (start 135.8 134.6) (end 135.8 129.365686) (width 0.2) (layer "F.Cu") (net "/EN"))
 (segment (start 121.06 143.5) (end 124.76 139.8) (width 0.2) (layer "F.Cu") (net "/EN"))
 (segment (start 128.965686 139.8) (end 133.965686 134.8) (width 0.2) (layer "F.Cu") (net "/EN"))
 (segment (start 109.8 135.365686) (end 108.965685 136.2) (width 0.2) (layer "F.Cu") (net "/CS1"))
 (segment (start 109.8 131) (end 109.8 135.365686) (width 0.2) (layer "F.Cu") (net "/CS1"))
 (segment (start 115.315881 84.87) (end 115.315881 125.484119) (width 0.2) (layer "F.Cu") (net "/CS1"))
 (segment (start 105.5 136.2) (end 98.2 143.5) (width 0.2) (layer "F.Cu") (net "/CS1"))
 (segment (start 115.315881 125.484119) (end 109.8 131) (width 0.2) (layer "F.Cu") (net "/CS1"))
 (segment (start 108.965685 136.2) (end 105.5 136.2) (width 0.2) (layer "F.Cu") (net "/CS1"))
 (segment (start 109.4 135.2) (end 108.8 135.8) (width 0.2) (layer "F.Cu") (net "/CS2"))
 (segment (start 112.775881 84.87) (end 112.775881 127.458433) (width 0.2) (layer "F.Cu") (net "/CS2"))
 (segment (start 103.36 135.8) (end 95.66 143.5) (width 0.2) (layer "F.Cu") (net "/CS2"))
 (segment (start 112.775881 127.458433) (end 109.4 130.834314) (width 0.2) (layer "F.Cu") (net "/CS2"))
 (segment (start 109.4 130.834314) (end 109.4 135.2) (width 0.2) (layer "F.Cu") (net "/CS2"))
 (segment (start 108.8 135.8) (end 103.36 135.8) (width 0.2) (layer "F.Cu") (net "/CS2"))
 (segment (start 124.459881 133.13) (end 126.999881 133.13) (width 0.2) (layer "F.Cu") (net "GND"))
 (segment (start 105.4 89.6) (end 110.13 84.87) (width 0.2) (layer "F.Cu") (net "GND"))
 (segment (start 98.37601 94.97601) (end 97.6 94.2) (width 0.2) (layer "F.Cu") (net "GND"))
 (segment (start 98.4 89.6) (end 105.4 89.6) (width 0.2) (layer "F.Cu") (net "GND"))
 (segment (start 100.075881 123.124119) (end 85.6 137.6) (width 0.2) (layer "F.Cu") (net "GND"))
 (segment (start 85.6 143.4) (end 85.5 143.5) (width 0.2) (layer "F.Cu") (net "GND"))
 (segment (start 97.6 90.4) (end 98.4 89.6) (width 0.2) (layer "F.Cu") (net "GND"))
 (segment (start 97.6 94.2) (end 97.6 90.4) (width 0.2) (layer "F.Cu") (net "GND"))
 (segment (start 100.075881 94.97601) (end 100.075881 123.124119) (width 0.2) (layer "F.Cu") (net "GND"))
 (segment (start 85.6 137.6) (end 85.6 143.4) (width 0.2) (layer "F.Cu") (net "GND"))
 (segment (start 100.075881 94.97601) (end 98.37601 94.97601) (width 0.2) (layer "F.Cu") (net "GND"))
 (segment (start 110.13 84.87) (end 110.235881 84.87) (width 0.2) (layer "F.Cu") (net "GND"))
 (segment (start 160.8 121.083119) (end 149.986881 110.27) (width 0.2) (layer "B.Cu") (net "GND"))
 (segment (start 124.459881 142.640119) (end 124.459881 139) (width 0.2) (layer "B.Cu") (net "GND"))
 (segment (start 90 139) (end 124.459881 139) (width 0.2) (layer "B.Cu") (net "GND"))
 (segment (start 124.459881 139) (end 124.459881 133.13) (width 0.2) (layer "B.Cu") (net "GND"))
 (segment (start 157.01 124.79) (end 154.8 127) (width 0.2) (layer "B.Cu") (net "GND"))
 (segment (start 160.8 124.79) (end 160.8 121.083119) (width 0.2) (layer "B.Cu") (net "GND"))
 (segment (start 160.8 124.79) (end 157.01 124.79) (width 0.2) (layer "B.Cu") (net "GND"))
 (segment (start 85.5 143.5) (end 90 139) (width 0.2) (layer "B.Cu") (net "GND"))
 (segment (start 123.6 143.5) (end 124.459881 142.640119) (width 0.2) (layer "B.Cu") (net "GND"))
 (segment (start 154.8 139) (end 150.3 143.5) (width 0.2) (layer "B.Cu") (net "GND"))
 (segment (start 133.76 139.890119) (end 126.999881 133.13) (width 0.2) (layer "B.Cu") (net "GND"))
 (segment (start 133.76 143.5) (end 133.76 139.890119) (width 0.2) (layer "B.Cu") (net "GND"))
 (segment (start 150.3 143.5) (end 133.76 143.5) (width 0.2) (layer "B.Cu") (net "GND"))
 (segment (start 154.8 127) (end 154.8 139) (width 0.2) (layer "B.Cu") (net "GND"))
 (segment (start 105.285881 82.2) (end 102.615881 84.87) (width 0.2) (layer "F.Cu") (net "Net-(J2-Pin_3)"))
 (segment (start 111.4 82.2) (end 105.285881 82.2) (width 0.2) (layer "F.Cu") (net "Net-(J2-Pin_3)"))
 (via (at 111.4 82.2) (size 0.6) (drill 0.3) (layers "F.Cu" "B.Cu") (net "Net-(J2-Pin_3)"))
 (segment (start 160.8 129.87) (end 163 127.67) (width 0.2) (layer "B.Cu") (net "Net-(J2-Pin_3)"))
 (segment (start 162.134314 82.8) (end 152.4 82.8) (width 0.2) (layer "B.Cu") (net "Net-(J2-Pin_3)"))
 (segment (start 163 127.67) (end 163 83.665686) (width 0.2) (layer "B.Cu") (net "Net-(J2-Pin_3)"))
 (segment (start 152.4 82.8) (end 150.2 80.6) (width 0.2) (layer "B.Cu") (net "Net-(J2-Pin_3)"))
 (segment (start 113 80.6) (end 111.4 82.2) (width 0.2) (layer "B.Cu") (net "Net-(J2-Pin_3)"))
 (segment (start 163 83.665686) (end 162.134314 82.8) (width 0.2) (layer "B.Cu") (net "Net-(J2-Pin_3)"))
 (segment (start 150.2 80.6) (end 113 80.6) (width 0.2) (layer "B.Cu") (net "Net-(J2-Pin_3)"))
 (segment (start 163.4 129.81) (end 163.4 83.5) (width 0.2) (layer "B.Cu") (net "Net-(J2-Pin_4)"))
 (segment (start 162.3 82.4) (end 152.6 82.4) (width 0.2) (layer "B.Cu") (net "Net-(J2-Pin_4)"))
 (segment (start 160.8 132.41) (end 163.4 129.81) (width 0.2) (layer "B.Cu") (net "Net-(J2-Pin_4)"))
 (segment (start 163.4 83.5) (end 162.3 82.4) (width 0.2) (layer "B.Cu") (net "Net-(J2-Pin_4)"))
 (segment (start 152.6 82.4) (end 150.4 80.2) (width 0.2) (layer "B.Cu") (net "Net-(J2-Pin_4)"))
 (segment (start 150.4 80.2) (end 109.825881 80.2) (width 0.2) (layer "B.Cu") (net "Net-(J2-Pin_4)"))
 (segment (start 109.825881 80.2) (end 105.155881 84.87) (width 0.2) (layer "B.Cu") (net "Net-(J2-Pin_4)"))
 (segment (start 145 125.8) (end 145 98.2) (width 0.2) (layer "F.Cu") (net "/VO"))
 (segment (start 154.1 94.8) (end 157.5 91.4) (width 0.2) (layer "F.Cu") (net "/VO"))
 (segment (start 138.4 132.4) (end 145 125.8) (width 0.2) (layer "F.Cu") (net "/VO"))
 (segment (start 128.68 143.5) (end 130 142.18) (width 0.2) (layer "F.Cu") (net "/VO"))
 (segment (start 148.4 94.8) (end 154.1 94.8) (width 0.2) (layer "F.Cu") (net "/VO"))
 (segment (start 130.02 142.18) (end 138.4 133.8) (width 0.2) (layer "F.Cu") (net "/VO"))
 (segment (start 130 142.18) (end 130.02 142.18) (width 0.2) (layer "F.Cu") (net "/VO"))
 (segment (start 145 98.2) (end 148.4 94.8) (width 0.2) (layer "F.Cu") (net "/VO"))
 (segment (start 138.4 133.8) (end 138.4 132.4) (width 0.2) (layer "F.Cu") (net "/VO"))
 (segment (start 90.6 135.6) (end 90.58 135.62) (width 0.2) (layer "F.Cu") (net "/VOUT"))
 (segment (start 90.6 134.6) (end 90.6 135.6) (width 0.2) (layer "F.Cu") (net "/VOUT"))
 (segment (start 126.4 111.8) (end 126.4 123) (width 0.2) (layer "F.Cu") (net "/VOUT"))
 (segment (start 90.58 135.62) (end 90.58 143.5) (width 0.2) (layer "F.Cu") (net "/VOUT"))
 (segment (start 128.5 109.7) (end 126.4 111.8) (width 0.2) (layer "F.Cu") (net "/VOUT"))
 (via (at 128.5 109.7) (size 0.6) (drill 0.3) (layers "F.Cu" "B.Cu") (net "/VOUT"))
 (via (at 90.6 134.6) (size 0.6) (drill 0.3) (layers "F.Cu" "B.Cu") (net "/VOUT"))
 (via (at 126.4 123) (size 0.6) (drill 0.3) (layers "F.Cu" "B.Cu") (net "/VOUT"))
 (segment (start 153.6 84.6) (end 158.2 84.6) (width 0.2) (layer "B.Cu") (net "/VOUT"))
 (segment (start 96.4 128.8) (end 120.6 128.8) (width 0.2) (layer "B.Cu") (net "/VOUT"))
 (segment (start 128.5 109.7) (end 153.6 84.6) (width 0.2) (layer "B.Cu") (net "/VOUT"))
 (segment (start 120.6 128.8) (end 126.4 123) (width 0.2) (layer "B.Cu") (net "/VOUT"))
 (segment (start 158.2 84.6) (end 160 86.4) (width 0.2) (layer "B.Cu") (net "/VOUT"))
 (segment (start 90.6 134.6) (end 96.4 128.8) (width 0.2) (layer "B.Cu") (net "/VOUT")))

